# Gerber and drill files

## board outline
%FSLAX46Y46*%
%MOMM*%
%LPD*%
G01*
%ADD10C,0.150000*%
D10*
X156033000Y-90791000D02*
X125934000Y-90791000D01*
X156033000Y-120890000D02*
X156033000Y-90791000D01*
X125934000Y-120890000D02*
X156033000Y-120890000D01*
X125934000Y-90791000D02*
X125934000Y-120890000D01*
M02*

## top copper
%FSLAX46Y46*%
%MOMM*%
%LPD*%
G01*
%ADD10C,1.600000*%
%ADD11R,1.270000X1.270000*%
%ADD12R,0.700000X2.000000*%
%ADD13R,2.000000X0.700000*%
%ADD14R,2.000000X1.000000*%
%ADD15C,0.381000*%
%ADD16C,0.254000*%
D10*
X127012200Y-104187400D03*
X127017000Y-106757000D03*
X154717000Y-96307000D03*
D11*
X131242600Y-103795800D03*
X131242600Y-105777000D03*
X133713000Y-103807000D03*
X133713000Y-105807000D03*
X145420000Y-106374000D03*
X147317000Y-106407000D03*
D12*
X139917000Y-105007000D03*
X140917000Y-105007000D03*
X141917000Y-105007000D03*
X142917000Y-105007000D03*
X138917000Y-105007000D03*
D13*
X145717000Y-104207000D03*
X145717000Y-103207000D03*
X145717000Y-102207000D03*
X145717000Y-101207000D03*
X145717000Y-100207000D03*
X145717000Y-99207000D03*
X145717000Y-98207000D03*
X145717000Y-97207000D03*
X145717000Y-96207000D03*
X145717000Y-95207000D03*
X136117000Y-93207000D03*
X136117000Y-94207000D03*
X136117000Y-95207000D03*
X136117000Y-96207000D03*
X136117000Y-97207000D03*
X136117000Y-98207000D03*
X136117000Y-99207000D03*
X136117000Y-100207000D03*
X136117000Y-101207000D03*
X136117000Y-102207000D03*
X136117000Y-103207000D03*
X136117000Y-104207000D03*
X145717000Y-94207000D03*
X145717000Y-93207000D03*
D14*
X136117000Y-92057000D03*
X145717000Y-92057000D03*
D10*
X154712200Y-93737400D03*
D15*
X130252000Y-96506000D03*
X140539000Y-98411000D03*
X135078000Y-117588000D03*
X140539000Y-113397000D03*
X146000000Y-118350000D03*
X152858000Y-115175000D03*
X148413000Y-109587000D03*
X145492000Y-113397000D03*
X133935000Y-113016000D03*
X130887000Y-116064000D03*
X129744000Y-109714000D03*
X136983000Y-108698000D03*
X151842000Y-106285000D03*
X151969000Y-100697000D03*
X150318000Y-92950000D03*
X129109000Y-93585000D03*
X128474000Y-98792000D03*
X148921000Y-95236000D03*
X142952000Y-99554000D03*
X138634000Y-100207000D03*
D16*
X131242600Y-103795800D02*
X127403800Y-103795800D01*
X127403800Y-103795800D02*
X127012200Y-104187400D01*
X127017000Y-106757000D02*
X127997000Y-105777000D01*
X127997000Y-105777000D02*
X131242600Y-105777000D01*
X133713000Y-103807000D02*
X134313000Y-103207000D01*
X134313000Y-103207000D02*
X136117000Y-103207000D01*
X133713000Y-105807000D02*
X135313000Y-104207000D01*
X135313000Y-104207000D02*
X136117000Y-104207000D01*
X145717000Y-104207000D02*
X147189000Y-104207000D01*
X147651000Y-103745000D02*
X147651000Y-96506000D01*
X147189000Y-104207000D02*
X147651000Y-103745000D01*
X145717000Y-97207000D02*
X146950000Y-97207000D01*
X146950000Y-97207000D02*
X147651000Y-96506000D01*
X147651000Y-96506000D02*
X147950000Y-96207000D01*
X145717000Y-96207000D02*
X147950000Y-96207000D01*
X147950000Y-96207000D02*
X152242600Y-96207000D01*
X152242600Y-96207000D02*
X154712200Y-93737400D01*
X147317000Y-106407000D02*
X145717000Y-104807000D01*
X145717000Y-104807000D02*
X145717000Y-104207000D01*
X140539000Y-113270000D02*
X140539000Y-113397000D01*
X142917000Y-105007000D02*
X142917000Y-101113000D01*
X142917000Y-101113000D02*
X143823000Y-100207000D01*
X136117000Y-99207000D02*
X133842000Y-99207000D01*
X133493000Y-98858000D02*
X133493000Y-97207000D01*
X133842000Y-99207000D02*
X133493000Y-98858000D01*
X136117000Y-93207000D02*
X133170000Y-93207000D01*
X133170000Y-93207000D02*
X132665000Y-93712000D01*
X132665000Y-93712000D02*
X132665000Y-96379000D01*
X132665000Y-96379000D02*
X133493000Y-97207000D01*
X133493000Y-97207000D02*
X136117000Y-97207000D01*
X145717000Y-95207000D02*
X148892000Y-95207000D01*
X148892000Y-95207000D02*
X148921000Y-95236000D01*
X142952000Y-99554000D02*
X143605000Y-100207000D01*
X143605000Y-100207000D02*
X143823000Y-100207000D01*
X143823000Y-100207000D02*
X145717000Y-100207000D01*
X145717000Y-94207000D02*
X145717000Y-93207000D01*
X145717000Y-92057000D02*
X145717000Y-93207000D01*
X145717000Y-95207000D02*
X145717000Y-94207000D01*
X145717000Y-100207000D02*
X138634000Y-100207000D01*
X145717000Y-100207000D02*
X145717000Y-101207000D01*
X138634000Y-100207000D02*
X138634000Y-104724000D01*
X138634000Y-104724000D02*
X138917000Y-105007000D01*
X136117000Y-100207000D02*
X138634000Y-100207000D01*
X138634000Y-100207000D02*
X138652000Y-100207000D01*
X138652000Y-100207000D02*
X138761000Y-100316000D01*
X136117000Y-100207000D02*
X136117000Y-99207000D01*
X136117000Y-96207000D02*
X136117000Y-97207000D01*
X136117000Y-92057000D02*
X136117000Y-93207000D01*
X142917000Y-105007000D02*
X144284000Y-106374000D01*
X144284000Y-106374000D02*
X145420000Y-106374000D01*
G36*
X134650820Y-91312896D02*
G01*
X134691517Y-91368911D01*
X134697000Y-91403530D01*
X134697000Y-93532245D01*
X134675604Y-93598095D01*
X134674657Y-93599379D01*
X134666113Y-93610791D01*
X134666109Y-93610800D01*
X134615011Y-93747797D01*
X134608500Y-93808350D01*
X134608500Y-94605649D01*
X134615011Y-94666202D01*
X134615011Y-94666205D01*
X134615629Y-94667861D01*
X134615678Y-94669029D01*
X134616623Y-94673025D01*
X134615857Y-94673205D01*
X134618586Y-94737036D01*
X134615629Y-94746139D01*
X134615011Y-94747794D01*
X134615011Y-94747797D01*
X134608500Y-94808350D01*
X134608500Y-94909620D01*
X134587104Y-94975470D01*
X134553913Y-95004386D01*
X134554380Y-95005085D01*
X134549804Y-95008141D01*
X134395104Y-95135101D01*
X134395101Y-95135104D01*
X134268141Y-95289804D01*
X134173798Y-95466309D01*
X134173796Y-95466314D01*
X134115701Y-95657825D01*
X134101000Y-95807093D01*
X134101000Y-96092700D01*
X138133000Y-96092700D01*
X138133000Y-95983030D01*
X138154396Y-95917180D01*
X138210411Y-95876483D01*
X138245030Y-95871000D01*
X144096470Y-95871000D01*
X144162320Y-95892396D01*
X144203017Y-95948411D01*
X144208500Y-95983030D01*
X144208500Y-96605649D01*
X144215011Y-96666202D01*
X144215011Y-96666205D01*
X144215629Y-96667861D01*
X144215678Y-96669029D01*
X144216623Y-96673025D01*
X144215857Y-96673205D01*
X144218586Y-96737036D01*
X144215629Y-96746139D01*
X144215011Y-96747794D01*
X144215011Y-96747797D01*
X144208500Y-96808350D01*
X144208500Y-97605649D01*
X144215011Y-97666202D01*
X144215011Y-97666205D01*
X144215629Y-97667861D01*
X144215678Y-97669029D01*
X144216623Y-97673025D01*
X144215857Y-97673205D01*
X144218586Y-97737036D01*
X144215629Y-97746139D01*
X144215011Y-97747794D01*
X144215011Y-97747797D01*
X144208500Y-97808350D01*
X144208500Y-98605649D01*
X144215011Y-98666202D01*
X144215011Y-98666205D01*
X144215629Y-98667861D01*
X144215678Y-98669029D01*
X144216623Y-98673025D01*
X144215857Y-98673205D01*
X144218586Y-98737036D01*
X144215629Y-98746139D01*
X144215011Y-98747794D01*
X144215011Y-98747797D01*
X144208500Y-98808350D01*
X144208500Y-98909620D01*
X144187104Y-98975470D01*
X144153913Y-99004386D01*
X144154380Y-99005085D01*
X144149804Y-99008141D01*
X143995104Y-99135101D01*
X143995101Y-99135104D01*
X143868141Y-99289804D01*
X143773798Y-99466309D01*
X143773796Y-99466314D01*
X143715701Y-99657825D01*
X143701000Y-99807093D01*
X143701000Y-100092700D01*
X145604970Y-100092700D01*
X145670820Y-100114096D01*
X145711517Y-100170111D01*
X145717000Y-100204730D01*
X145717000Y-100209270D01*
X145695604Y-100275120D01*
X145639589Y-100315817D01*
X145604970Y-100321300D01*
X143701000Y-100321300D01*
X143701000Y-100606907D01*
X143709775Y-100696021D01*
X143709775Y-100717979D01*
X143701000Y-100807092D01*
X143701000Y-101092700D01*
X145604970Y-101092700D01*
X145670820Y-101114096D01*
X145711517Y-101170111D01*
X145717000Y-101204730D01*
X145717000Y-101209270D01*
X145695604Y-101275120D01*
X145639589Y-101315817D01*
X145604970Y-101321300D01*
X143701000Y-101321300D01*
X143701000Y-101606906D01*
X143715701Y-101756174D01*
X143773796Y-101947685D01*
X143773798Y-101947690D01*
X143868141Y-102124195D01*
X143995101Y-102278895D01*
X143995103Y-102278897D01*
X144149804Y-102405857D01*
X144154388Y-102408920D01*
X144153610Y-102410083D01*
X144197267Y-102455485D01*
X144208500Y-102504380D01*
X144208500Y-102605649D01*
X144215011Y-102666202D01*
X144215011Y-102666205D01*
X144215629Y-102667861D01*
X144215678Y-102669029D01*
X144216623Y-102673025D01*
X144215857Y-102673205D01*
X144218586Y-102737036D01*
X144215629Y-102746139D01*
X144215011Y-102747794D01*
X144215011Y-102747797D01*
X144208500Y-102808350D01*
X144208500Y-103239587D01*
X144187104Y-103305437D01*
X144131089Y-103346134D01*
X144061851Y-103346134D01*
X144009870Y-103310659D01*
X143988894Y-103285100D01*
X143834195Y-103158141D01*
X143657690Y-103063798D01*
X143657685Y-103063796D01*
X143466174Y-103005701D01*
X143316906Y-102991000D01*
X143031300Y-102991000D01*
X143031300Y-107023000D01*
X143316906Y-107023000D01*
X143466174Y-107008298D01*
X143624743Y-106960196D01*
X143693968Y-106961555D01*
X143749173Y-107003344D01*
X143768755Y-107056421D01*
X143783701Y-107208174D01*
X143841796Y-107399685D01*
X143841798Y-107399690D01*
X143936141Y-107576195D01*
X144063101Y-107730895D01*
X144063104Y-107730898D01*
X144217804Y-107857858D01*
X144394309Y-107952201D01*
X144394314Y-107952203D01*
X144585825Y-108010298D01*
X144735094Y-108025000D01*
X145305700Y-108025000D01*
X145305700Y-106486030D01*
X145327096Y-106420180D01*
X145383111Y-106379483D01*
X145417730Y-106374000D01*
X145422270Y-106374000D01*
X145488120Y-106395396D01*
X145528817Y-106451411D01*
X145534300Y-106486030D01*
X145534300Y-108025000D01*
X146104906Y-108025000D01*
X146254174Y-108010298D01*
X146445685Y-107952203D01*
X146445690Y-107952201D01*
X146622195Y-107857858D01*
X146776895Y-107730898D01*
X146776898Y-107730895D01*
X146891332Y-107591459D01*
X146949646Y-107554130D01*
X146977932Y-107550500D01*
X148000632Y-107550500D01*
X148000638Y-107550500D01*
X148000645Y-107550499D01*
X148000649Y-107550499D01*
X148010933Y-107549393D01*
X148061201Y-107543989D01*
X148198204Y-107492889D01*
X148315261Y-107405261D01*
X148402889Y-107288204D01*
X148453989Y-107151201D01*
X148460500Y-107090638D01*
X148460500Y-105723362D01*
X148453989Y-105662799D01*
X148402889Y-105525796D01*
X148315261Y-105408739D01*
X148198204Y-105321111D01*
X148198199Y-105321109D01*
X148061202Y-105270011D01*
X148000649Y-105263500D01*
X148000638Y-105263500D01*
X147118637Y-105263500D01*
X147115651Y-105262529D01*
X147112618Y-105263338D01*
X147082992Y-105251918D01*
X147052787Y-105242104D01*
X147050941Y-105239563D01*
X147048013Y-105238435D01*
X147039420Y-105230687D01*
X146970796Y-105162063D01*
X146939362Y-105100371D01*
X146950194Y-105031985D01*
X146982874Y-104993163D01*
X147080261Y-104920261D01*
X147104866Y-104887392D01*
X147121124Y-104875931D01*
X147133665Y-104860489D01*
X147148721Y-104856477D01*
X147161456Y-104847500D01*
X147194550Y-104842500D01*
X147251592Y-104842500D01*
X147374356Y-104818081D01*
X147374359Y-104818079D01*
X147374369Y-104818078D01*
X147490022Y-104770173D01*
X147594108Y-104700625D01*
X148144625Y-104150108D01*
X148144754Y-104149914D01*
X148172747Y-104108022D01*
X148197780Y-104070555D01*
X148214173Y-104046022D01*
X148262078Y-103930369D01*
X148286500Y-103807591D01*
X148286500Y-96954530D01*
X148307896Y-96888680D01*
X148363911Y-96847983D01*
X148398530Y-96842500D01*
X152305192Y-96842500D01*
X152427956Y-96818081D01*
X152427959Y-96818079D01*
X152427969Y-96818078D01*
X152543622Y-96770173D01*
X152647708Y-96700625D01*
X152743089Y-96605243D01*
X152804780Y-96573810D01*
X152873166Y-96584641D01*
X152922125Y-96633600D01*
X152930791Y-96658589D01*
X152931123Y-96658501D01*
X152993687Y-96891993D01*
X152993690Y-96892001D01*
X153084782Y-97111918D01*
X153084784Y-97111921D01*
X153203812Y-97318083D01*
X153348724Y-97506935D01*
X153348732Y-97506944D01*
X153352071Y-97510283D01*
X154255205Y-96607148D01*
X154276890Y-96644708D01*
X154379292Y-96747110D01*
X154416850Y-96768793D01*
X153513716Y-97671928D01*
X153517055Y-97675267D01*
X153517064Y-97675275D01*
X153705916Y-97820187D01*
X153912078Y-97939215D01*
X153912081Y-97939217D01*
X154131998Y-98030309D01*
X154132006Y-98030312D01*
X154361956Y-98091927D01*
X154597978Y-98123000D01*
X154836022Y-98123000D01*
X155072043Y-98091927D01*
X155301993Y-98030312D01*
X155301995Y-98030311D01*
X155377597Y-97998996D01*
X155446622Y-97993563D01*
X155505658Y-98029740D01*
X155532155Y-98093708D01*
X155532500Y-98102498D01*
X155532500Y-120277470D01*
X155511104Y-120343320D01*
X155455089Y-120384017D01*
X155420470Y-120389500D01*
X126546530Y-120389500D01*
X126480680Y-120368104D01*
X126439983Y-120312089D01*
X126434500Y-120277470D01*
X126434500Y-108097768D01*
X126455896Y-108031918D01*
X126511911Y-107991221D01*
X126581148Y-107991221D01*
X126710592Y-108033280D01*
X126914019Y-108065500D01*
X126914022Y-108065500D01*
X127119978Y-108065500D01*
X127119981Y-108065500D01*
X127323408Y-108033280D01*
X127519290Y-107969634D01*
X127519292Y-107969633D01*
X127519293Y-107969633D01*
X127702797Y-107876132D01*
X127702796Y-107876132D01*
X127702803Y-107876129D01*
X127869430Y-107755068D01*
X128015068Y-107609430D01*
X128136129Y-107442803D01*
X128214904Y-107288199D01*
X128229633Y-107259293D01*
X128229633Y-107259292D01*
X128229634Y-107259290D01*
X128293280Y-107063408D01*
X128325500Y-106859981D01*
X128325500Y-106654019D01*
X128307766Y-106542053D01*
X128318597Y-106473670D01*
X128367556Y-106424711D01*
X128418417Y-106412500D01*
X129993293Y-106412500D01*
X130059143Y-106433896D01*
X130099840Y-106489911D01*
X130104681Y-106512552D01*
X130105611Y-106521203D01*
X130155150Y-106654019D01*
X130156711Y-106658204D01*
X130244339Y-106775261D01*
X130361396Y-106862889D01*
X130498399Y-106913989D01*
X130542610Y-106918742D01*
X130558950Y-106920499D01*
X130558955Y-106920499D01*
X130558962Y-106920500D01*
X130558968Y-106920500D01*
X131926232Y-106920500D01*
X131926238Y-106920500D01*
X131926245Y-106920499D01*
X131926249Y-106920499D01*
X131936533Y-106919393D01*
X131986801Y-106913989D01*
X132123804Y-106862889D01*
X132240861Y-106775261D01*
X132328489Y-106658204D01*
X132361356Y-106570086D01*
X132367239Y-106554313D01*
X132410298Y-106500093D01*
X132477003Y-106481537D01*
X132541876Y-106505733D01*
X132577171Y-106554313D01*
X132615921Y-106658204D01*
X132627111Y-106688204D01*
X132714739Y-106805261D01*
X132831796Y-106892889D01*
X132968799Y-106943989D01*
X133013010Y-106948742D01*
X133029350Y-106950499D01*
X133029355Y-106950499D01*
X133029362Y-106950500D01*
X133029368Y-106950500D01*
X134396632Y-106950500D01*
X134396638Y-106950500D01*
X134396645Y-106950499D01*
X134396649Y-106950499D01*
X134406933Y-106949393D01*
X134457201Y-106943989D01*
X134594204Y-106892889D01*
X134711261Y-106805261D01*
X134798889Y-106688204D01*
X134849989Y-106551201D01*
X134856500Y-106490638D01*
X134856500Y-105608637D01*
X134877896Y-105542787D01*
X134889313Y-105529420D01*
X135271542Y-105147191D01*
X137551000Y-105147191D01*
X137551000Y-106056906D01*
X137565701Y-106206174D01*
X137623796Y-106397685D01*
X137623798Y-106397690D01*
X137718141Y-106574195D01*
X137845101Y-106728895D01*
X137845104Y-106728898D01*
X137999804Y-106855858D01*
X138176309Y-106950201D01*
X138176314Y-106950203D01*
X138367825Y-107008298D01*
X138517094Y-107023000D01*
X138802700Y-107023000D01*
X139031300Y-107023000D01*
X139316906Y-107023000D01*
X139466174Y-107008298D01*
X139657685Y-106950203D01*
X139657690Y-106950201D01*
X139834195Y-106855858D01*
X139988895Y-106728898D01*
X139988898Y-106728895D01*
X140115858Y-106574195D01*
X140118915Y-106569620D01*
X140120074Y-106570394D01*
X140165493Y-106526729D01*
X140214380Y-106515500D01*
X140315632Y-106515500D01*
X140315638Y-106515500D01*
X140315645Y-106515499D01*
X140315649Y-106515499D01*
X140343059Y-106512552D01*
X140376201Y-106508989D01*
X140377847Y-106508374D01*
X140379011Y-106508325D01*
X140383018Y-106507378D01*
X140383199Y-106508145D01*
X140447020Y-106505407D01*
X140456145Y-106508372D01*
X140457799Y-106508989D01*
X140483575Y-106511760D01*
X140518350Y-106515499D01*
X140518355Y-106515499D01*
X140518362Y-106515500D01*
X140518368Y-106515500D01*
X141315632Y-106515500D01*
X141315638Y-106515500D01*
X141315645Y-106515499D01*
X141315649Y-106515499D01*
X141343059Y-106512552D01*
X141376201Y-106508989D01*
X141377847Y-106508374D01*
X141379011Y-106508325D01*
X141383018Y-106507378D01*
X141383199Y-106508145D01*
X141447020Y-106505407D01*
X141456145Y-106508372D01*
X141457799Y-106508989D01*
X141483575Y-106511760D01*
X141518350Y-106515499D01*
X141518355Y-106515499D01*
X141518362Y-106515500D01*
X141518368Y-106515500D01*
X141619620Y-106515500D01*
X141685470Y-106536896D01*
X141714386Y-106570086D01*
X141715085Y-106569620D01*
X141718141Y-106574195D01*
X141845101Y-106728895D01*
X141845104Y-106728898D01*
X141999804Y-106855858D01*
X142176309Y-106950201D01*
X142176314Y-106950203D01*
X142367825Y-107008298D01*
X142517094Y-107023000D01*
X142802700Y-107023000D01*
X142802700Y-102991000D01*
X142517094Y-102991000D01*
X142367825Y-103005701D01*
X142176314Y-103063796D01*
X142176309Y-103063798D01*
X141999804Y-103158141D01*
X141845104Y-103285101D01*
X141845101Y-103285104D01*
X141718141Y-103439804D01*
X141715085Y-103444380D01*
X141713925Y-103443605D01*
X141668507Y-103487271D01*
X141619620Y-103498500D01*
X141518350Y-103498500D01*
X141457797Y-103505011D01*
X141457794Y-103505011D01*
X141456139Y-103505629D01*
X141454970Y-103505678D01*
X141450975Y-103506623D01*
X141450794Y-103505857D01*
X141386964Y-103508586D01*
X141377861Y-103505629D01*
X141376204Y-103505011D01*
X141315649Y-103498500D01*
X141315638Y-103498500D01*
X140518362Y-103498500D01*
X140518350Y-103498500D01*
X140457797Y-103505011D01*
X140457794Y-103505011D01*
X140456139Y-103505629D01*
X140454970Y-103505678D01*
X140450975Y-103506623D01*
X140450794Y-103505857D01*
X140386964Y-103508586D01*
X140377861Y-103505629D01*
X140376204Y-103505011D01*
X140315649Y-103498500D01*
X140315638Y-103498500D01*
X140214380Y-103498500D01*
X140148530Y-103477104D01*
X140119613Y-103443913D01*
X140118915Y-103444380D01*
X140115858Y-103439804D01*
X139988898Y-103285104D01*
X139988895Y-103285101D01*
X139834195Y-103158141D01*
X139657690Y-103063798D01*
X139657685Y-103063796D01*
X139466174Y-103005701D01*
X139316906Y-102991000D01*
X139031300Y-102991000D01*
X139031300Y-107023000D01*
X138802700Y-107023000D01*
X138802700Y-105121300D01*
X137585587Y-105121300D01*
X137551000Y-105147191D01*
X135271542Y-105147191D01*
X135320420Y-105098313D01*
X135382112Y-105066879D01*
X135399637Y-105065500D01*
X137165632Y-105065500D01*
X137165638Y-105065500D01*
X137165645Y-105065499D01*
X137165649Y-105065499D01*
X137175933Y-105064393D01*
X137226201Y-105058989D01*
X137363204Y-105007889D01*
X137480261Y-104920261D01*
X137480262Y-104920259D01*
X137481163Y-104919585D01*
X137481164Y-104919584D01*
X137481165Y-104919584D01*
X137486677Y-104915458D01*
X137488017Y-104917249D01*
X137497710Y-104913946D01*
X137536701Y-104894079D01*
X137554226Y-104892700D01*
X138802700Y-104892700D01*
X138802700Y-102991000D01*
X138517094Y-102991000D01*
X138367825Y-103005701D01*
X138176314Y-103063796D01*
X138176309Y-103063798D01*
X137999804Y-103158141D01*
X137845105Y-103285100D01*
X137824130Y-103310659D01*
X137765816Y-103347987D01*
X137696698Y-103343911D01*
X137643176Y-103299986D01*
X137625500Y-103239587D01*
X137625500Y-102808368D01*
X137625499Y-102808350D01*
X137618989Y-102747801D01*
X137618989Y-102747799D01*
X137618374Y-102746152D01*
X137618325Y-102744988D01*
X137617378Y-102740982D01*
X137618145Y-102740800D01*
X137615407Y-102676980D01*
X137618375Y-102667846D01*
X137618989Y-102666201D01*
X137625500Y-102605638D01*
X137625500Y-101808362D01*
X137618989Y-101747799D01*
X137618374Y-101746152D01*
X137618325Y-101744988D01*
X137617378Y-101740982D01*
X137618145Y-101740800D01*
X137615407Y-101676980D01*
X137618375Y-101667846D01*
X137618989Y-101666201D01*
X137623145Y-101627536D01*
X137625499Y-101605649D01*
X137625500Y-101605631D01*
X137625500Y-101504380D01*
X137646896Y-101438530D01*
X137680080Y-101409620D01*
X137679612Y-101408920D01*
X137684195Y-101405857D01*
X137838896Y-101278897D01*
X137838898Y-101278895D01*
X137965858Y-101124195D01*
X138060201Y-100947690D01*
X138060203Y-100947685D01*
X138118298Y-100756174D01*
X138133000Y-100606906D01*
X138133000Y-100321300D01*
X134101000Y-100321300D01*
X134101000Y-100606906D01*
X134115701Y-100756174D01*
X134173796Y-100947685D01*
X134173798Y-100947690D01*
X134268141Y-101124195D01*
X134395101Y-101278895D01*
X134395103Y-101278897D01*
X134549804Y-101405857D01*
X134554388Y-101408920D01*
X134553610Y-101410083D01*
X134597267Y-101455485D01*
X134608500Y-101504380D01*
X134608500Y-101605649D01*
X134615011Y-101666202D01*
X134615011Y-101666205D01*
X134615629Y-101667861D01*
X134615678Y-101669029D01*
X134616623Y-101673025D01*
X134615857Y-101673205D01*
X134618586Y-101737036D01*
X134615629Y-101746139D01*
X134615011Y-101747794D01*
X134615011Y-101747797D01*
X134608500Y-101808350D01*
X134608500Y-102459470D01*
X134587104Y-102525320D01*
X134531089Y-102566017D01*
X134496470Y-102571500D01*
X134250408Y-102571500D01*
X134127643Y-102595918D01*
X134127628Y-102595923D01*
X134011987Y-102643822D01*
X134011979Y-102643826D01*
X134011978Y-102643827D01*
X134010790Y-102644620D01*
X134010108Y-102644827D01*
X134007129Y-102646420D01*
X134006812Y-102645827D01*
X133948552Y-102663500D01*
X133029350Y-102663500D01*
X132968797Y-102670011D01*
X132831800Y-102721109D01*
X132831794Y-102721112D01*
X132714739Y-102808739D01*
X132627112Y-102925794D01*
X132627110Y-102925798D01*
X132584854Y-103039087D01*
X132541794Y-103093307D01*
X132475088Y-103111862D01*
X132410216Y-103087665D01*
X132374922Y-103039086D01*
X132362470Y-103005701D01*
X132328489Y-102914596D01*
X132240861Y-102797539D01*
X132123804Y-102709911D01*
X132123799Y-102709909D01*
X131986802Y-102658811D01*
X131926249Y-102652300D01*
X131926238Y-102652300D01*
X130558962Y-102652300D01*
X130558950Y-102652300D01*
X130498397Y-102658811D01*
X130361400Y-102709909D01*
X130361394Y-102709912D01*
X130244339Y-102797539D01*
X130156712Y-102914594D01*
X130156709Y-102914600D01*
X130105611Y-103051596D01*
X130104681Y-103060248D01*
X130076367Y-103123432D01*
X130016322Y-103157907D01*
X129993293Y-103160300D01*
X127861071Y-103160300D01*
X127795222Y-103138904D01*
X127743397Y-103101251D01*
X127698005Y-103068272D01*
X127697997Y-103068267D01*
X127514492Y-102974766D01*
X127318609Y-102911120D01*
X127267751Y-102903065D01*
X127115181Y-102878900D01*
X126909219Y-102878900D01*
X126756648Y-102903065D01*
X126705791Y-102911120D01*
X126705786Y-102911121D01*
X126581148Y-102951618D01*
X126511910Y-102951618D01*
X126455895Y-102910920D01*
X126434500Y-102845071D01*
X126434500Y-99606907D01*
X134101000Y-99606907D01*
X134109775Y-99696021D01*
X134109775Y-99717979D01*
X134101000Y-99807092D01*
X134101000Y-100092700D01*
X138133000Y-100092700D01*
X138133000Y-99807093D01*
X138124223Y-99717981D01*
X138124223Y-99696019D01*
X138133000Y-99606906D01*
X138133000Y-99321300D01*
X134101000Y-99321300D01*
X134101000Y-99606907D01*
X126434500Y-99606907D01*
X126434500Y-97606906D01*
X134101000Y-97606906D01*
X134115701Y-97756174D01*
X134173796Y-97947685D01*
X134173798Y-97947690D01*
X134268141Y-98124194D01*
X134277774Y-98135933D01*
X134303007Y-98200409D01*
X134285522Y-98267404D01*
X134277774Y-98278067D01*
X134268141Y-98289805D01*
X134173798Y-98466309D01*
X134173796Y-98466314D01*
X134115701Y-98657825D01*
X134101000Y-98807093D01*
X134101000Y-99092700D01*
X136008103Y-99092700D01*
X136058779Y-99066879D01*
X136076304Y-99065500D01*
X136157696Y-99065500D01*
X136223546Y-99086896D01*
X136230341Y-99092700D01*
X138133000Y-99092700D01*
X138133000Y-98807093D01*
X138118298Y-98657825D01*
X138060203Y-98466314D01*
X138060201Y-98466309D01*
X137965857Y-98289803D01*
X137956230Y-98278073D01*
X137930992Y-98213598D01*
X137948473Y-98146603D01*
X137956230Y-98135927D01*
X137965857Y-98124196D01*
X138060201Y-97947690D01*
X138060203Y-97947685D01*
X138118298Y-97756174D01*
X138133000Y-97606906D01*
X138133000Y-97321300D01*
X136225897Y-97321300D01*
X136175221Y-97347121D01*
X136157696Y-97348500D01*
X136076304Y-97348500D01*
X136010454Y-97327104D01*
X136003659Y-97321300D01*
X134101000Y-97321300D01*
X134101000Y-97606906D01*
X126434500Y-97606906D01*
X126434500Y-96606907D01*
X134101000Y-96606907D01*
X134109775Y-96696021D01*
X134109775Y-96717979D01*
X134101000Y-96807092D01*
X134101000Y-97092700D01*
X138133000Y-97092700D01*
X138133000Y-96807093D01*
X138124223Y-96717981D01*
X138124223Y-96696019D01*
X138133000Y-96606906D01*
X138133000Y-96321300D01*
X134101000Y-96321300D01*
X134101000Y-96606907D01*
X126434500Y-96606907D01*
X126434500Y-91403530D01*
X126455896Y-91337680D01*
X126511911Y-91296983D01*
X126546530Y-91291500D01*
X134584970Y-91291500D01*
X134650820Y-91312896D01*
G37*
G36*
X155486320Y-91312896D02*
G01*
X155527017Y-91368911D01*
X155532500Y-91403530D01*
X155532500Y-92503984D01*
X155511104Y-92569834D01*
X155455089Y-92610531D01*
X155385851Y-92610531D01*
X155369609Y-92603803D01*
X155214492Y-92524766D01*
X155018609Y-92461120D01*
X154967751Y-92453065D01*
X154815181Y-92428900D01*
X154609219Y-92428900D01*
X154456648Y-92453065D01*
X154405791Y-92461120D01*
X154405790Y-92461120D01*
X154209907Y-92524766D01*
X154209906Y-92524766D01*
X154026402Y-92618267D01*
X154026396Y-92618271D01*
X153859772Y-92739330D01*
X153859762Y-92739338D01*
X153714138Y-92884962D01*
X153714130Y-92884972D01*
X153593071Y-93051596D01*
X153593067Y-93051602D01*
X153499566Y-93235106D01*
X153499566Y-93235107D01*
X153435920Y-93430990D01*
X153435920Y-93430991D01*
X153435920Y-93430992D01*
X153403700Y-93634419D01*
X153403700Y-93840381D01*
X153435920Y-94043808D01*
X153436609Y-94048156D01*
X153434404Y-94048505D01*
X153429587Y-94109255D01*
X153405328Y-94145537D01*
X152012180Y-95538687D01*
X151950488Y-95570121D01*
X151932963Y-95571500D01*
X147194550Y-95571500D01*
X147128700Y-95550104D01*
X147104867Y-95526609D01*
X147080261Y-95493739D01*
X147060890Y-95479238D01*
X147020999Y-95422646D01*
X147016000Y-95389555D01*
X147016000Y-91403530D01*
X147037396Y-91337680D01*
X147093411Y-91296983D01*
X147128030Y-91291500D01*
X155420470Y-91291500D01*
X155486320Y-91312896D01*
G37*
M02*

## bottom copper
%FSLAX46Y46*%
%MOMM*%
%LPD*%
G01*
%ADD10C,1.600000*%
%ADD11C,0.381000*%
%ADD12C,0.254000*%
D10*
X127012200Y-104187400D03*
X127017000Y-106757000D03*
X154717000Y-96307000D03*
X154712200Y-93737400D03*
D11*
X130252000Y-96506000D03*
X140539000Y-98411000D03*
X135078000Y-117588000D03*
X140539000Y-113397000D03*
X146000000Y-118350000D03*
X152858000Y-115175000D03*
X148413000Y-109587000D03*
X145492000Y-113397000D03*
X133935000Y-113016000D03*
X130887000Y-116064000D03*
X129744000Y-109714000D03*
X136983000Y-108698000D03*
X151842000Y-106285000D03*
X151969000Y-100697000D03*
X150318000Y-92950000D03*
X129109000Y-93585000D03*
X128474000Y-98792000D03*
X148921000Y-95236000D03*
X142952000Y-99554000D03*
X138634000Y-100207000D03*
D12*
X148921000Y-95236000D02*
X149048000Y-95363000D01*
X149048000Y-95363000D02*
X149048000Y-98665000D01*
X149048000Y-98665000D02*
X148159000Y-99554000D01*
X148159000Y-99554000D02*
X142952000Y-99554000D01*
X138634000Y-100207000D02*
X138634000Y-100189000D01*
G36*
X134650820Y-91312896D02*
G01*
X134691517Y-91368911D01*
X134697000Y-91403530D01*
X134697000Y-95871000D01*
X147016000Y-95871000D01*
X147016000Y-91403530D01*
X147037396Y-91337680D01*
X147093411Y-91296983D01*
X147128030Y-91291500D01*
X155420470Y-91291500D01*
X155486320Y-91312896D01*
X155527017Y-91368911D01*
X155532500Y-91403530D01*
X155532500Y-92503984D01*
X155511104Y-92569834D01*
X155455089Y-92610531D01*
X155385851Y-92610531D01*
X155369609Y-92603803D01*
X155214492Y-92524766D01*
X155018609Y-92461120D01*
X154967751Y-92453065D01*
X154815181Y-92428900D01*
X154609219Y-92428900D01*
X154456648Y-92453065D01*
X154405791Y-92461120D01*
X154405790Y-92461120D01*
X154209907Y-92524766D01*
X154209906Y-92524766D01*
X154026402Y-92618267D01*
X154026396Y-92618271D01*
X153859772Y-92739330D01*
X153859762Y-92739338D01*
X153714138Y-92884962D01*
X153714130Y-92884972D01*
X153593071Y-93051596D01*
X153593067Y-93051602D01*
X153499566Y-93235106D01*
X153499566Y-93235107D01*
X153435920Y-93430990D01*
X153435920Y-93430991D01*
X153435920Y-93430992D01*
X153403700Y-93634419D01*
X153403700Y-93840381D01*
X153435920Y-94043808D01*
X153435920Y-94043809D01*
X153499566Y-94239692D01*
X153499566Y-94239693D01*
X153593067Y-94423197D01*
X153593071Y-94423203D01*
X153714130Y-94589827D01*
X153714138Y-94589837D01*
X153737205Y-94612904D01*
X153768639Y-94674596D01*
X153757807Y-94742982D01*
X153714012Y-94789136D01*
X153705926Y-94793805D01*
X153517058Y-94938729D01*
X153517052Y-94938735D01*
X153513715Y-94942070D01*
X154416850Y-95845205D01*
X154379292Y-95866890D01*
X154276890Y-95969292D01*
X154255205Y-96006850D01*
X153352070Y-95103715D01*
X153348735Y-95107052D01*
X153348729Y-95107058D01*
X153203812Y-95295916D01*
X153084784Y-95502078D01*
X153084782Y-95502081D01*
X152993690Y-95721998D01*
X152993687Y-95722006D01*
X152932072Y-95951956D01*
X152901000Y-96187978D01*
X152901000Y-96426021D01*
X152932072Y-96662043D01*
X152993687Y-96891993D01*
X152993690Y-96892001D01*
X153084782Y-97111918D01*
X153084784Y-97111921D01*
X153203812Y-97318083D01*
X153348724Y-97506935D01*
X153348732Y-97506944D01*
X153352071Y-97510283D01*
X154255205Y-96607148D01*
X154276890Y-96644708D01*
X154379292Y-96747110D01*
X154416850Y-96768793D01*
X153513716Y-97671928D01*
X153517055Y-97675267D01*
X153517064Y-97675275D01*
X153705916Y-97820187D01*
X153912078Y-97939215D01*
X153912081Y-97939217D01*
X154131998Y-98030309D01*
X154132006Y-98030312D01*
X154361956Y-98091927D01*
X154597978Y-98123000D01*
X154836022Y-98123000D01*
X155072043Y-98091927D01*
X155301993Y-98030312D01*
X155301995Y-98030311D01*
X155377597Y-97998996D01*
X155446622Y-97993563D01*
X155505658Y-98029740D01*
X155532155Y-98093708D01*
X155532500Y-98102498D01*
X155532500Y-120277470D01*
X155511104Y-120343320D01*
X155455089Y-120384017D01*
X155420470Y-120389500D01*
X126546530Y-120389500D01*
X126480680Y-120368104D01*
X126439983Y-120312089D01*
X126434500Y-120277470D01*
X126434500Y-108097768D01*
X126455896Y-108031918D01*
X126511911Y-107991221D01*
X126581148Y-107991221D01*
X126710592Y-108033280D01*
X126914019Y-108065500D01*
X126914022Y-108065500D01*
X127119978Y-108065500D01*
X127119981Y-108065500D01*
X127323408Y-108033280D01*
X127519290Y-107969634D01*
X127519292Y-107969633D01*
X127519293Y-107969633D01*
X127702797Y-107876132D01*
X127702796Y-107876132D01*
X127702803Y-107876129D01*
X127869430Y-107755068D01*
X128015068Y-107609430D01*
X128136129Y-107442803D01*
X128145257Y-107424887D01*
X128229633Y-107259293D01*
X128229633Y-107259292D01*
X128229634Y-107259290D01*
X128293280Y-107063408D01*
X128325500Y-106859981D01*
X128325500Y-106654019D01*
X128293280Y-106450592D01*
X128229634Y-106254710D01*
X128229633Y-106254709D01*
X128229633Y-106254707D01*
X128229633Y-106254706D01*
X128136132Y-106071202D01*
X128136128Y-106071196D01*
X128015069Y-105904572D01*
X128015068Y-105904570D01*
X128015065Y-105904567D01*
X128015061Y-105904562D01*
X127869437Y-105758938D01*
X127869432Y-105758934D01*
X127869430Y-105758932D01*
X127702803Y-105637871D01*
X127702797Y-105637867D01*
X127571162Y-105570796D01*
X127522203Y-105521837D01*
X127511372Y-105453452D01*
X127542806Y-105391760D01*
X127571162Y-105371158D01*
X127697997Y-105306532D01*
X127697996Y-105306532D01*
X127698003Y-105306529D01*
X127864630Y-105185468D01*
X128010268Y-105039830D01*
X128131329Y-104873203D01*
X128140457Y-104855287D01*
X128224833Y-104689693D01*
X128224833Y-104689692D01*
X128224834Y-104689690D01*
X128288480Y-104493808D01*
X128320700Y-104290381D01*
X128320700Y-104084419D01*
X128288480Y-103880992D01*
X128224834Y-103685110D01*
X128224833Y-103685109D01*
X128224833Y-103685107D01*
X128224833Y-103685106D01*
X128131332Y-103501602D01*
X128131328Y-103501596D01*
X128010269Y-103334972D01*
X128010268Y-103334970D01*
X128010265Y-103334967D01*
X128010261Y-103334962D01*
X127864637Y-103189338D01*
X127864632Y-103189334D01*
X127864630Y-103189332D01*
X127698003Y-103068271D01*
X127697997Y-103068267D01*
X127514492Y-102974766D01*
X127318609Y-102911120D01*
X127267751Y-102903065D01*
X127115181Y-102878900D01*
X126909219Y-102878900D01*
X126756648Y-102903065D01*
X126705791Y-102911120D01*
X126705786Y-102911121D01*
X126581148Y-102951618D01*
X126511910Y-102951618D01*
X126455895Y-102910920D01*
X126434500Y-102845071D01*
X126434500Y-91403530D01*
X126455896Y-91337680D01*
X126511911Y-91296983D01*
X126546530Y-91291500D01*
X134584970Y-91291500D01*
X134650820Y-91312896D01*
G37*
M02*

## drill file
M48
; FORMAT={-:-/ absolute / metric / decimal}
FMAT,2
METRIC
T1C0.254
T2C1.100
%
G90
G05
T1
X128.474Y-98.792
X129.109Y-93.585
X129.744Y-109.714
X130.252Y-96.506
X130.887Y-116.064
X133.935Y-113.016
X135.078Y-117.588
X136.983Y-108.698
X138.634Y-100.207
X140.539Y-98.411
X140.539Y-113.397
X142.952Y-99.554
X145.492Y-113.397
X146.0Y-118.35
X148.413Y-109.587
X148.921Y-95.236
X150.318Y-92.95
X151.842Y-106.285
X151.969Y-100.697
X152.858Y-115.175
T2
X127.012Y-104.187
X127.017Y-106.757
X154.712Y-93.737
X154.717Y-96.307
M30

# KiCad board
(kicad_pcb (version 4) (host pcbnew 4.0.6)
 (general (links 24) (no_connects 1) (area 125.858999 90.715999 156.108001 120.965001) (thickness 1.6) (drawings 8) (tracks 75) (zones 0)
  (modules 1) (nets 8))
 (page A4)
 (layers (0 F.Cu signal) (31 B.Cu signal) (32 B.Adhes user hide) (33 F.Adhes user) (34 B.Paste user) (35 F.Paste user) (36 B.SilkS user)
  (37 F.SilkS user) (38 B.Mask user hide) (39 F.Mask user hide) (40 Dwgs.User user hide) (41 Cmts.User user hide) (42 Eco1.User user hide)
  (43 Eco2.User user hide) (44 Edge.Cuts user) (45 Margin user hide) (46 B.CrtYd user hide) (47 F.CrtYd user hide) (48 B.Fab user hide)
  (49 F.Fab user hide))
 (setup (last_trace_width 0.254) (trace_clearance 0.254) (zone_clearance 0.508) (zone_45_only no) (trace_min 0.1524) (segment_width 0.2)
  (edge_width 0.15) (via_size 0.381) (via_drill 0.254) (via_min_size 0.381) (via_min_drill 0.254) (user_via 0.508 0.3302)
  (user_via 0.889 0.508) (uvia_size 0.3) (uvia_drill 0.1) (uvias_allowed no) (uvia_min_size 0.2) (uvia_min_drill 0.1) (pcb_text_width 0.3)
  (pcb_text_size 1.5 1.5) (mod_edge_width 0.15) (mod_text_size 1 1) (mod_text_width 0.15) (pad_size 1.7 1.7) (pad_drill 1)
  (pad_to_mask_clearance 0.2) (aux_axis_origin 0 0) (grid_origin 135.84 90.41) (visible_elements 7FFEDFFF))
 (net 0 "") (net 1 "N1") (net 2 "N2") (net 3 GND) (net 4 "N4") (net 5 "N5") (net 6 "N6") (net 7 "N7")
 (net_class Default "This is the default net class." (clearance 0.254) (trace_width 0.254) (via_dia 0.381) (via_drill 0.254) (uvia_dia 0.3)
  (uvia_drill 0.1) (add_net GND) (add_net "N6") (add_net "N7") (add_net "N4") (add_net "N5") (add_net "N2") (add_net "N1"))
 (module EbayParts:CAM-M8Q (layer F.Cu) (at 135.967 91.807)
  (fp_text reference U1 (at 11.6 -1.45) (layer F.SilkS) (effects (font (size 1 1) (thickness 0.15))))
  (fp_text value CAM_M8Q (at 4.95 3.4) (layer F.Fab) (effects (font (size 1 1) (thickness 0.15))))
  (pad 62 thru_hole circle (at -8.9548 12.3804) (size 1.6 1.6) (drill 1.1) (layers *.Cu *.Mask) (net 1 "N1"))
  (pad 63 thru_hole circle (at -8.95 14.95) (size 1.6 1.6) (drill 1.1) (layers *.Cu *.Mask) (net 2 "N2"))
  (pad 61 thru_hole circle (at 18.75 4.5) (size 1.6 1.6) (drill 1.1) (layers *.Cu *.Mask) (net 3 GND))
  (pad 56 smd rect (at -4.7244 11.9888) (size 1.27 1.27) (layers F.Cu F.Paste F.Mask) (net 1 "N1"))
  (pad 54 smd rect (at -4.7244 13.97) (size 1.27 1.27) (layers F.Cu F.Paste F.Mask) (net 2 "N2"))
  (pad 55 smd rect (at -2.254 12) (size 1.27 1.27) (layers F.Cu F.Paste F.Mask) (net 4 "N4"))
  (pad 53 smd rect (at -2.254 14) (size 1.27 1.27) (layers F.Cu F.Paste F.Mask) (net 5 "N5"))
  (pad 50 smd rect (at 9.453 14.567) (size 1.27 1.27) (layers F.Cu F.Paste F.Mask) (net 3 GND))
  (pad 51 smd rect (at 11.35 14.6) (size 1.27 1.27) (layers F.Cu F.Paste F.Mask) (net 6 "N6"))
  (pad 28 smd rect (at 3.95 13.2) (size 0.7 2) (layers F.Cu F.Paste F.Mask))
  (pad 29 smd rect (at 4.95 13.2) (size 0.7 2) (layers F.Cu F.Paste F.Mask))
  (pad 30 smd rect (at 5.95 13.2) (size 0.7 2) (layers F.Cu F.Paste F.Mask))
  (pad 31 smd rect (at 6.95 13.2) (size 0.7 2) (layers F.Cu F.Paste F.Mask) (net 3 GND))
  (pad 27 smd rect (at 2.95 13.2) (size 0.7 2) (layers F.Cu F.Paste F.Mask) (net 3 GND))
  (pad 1 smd rect (at 9.75 12.4) (size 2 0.7) (layers F.Cu F.Paste F.Mask) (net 6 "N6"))
  (pad 2 smd rect (at 9.75 11.4) (size 2 0.7) (layers F.Cu F.Paste F.Mask))
  (pad 3 smd rect (at 9.75 10.4) (size 2 0.7) (layers F.Cu F.Paste F.Mask))
  (pad 4 smd rect (at 9.75 9.4) (size 2 0.7) (layers F.Cu F.Paste F.Mask) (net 3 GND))
  (pad 5 smd rect (at 9.75 8.4) (size 2 0.7) (layers F.Cu F.Paste F.Mask) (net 3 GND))
  (pad 6 smd rect (at 9.75 7.4) (size 2 0.7) (layers F.Cu F.Paste F.Mask))
  (pad 7 smd rect (at 9.75 6.4) (size 2 0.7) (layers F.Cu F.Paste F.Mask))
  (pad 8 smd rect (at 9.75 5.4) (size 2 0.7) (layers F.Cu F.Paste F.Mask) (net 6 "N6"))
  (pad 9 smd rect (at 9.75 4.4) (size 2 0.7) (layers F.Cu F.Paste F.Mask) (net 6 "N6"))
  (pad 10 smd rect (at 9.75 3.4) (size 2 0.7) (layers F.Cu F.Paste F.Mask) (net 3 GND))
  (pad 15 smd rect (at 0.15 1.4) (size 2 0.7) (layers F.Cu F.Paste F.Mask) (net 3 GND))
  (pad 16 smd rect (at 0.15 2.4) (size 2 0.7) (layers F.Cu F.Paste F.Mask) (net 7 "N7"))
  (pad 17 smd rect (at 0.15 3.4) (size 2 0.7) (layers F.Cu F.Paste F.Mask) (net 7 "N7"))
  (pad 18 smd rect (at 0.15 4.4) (size 2 0.7) (layers F.Cu F.Paste F.Mask) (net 3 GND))
  (pad 19 smd rect (at 0.15 5.4) (size 2 0.7) (layers F.Cu F.Paste F.Mask) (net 3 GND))
  (pad 20 smd rect (at 0.15 6.4) (size 2 0.7) (layers F.Cu F.Paste F.Mask))
  (pad 21 smd rect (at 0.15 7.4) (size 2 0.7) (layers F.Cu F.Paste F.Mask) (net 3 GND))
  (pad 22 smd rect (at 0.15 8.4) (size 2 0.7) (layers F.Cu F.Paste F.Mask) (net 3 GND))
  (pad 23 smd rect (at 0.15 9.4) (size 2 0.7) (layers F.Cu F.Paste F.Mask))
  (pad 24 smd rect (at 0.15 10.4) (size 2 0.7) (layers F.Cu F.Paste F.Mask))
  (pad 25 smd rect (at 0.15 11.4) (size 2 0.7) (layers F.Cu F.Paste F.Mask) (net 4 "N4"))
  (pad 26 smd rect (at 0.15 12.4) (size 2 0.7) (layers F.Cu F.Paste F.Mask) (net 5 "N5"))
  (pad 11 smd rect (at 9.75 2.4) (size 2 0.7) (layers F.Cu F.Paste F.Mask) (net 3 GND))
  (pad 12 smd rect (at 9.75 1.4) (size 2 0.7) (layers F.Cu F.Paste F.Mask) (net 3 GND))
  (pad 14 smd rect (at 0.15 0.25) (size 2 1) (layers F.Cu F.Paste F.Mask) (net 3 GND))
  (pad 13 smd rect (at 9.75 0.25) (size 2 1) (layers F.Cu F.Paste F.Mask) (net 3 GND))
  (pad 60 thru_hole circle (at 18.7452 1.9304) (size 1.6 1.6) (drill 1.1) (layers *.Cu *.Mask) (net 6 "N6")))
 (gr_line (start 156.033 90.791) (end 125.934 90.791) (angle 90) (layer Edge.Cuts) (width 0.15))
 (gr_line (start 156.033 120.89) (end 156.033 90.791) (angle 90) (layer Edge.Cuts) (width 0.15))
 (gr_line (start 125.934 120.89) (end 156.033 120.89) (angle 90) (layer Edge.Cuts) (width 0.15))
 (gr_line (start 125.934 90.791) (end 125.934 120.89) (angle 90) (layer Edge.Cuts) (width 0.15))
 (segment (start 131.2426 103.7958) (end 127.4038 103.7958) (width 0.254) (layer F.Cu) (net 1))
 (segment (start 127.4038 103.7958) (end 127.0122 104.1874) (width 0.254) (layer F.Cu) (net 1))
 (segment (start 127.017 106.757) (end 127.997 105.777) (width 0.254) (layer F.Cu) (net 2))
 (segment (start 127.997 105.777) (end 131.2426 105.777) (width 0.254) (layer F.Cu) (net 2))
 (segment (start 133.713 103.807) (end 134.313 103.207) (width 0.254) (layer F.Cu) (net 4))
 (segment (start 134.313 103.207) (end 136.117 103.207) (width 0.254) (layer F.Cu) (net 4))
 (segment (start 133.713 105.807) (end 135.313 104.207) (width 0.254) (layer F.Cu) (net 5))
 (segment (start 135.313 104.207) (end 136.117 104.207) (width 0.254) (layer F.Cu) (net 5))
 (segment (start 145.717 104.207) (end 147.189 104.207) (width 0.254) (layer F.Cu) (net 6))
 (segment (start 147.651 103.745) (end 147.651 96.506) (width 0.254) (layer F.Cu) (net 6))
 (segment (start 147.189 104.207) (end 147.651 103.745) (width 0.254) (layer F.Cu) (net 6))
 (segment (start 145.717 97.207) (end 146.95 97.207) (width 0.254) (layer F.Cu) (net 6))
 (segment (start 146.95 97.207) (end 147.651 96.506) (width 0.254) (layer F.Cu) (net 6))
 (segment (start 147.651 96.506) (end 147.95 96.207) (width 0.254) (layer F.Cu) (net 6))
 (segment (start 145.717 96.207) (end 147.95 96.207) (width 0.254) (layer F.Cu) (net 6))
 (segment (start 147.95 96.207) (end 152.2426 96.207) (width 0.254) (layer F.Cu) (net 6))
 (segment (start 152.2426 96.207) (end 154.7122 93.7374) (width 0.254) (layer F.Cu) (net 6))
 (segment (start 147.317 106.407) (end 145.717 104.807) (width 0.254) (layer F.Cu) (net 6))
 (segment (start 145.717 104.807) (end 145.717 104.207) (width 0.254) (layer F.Cu) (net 6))
 (via (at 130.252 96.506) (size 0.381) (drill 0.254) (layers F.Cu B.Cu) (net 3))
 (via (at 140.539 98.411) (size 0.381) (drill 0.254) (layers F.Cu B.Cu) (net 3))
 (via (at 135.078 117.588) (size 0.381) (drill 0.254) (layers F.Cu B.Cu) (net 3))
 (segment (start 140.539 113.27) (end 140.539 113.397) (width 0.254) (layer F.Cu) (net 3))
 (via (at 140.539 113.397) (size 0.381) (drill 0.254) (layers F.Cu B.Cu) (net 3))
 (via (at 146 118.35) (size 0.381) (drill 0.254) (layers F.Cu B.Cu) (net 3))
 (via (at 152.858 115.175) (size 0.381) (drill 0.254) (layers F.Cu B.Cu) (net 3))
 (via (at 148.413 109.587) (size 0.381) (drill 0.254) (layers F.Cu B.Cu) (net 3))
 (via (at 145.492 113.397) (size 0.381) (drill 0.254) (layers F.Cu B.Cu) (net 3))
 (via (at 133.935 113.016) (size 0.381) (drill 0.254) (layers F.Cu B.Cu) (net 3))
 (via (at 130.887 116.064) (size 0.381) (drill 0.254) (layers F.Cu B.Cu) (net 3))
 (via (at 129.744 109.714) (size 0.381) (drill 0.254) (layers F.Cu B.Cu) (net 3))
 (via (at 136.983 108.698) (size 0.381) (drill 0.254) (layers F.Cu B.Cu) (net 3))
 (via (at 151.842 106.285) (size 0.381) (drill 0.254) (layers F.Cu B.Cu) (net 3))
 (via (at 151.969 100.697) (size 0.381) (drill 0.254) (layers F.Cu B.Cu) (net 3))
 (via (at 150.318 92.95) (size 0.381) (drill 0.254) (layers F.Cu B.Cu) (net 3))
 (via (at 129.109 93.585) (size 0.381) (drill 0.254) (layers F.Cu B.Cu) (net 3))
 (via (at 128.474 98.792) (size 0.381) (drill 0.254) (layers F.Cu B.Cu) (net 3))
 (segment (start 142.917 105.007) (end 142.917 101.113) (width 0.254) (layer F.Cu) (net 3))
 (segment (start 142.917 101.113) (end 143.823 100.207) (width 0.254) (layer F.Cu) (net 3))
 (segment (start 136.117 99.207) (end 133.842 99.207) (width 0.254) (layer F.Cu) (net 3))
 (segment (start 133.493 98.858) (end 133.493 97.207) (width 0.254) (layer F.Cu) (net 3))
 (segment (start 133.842 99.207) (end 133.493 98.858) (width 0.254) (layer F.Cu) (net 3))
 (segment (start 136.117 93.207) (end 133.17 93.207) (width 0.254) (layer F.Cu) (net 3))
 (segment (start 133.17 93.207) (end 132.665 93.712) (width 0.254) (layer F.Cu) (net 3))
 (segment (start 132.665 93.712) (end 132.665 96.379) (width 0.254) (layer F.Cu) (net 3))
 (segment (start 132.665 96.379) (end 133.493 97.207) (width 0.254) (layer F.Cu) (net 3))
 (segment (start 133.493 97.207) (end 136.117 97.207) (width 0.254) (layer F.Cu) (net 3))
 (segment (start 145.717 95.207) (end 148.892 95.207) (width 0.254) (layer F.Cu) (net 3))
 (segment (start 148.892 95.207) (end 148.921 95.236) (width 0.254) (layer F.Cu) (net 3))
 (via (at 148.921 95.236) (size 0.381) (drill 0.254) (layers F.Cu B.Cu) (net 3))
 (segment (start 148.921 95.236) (end 149.048 95.363) (width 0.254) (layer B.Cu) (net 3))
 (segment (start 149.048 95.363) (end 149.048 98.665) (width 0.254) (layer B.Cu) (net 3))
 (segment (start 149.048 98.665) (end 148.159 99.554) (width 0.254) (layer B.Cu) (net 3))
 (segment (start 148.159 99.554) (end 142.952 99.554) (width 0.254) (layer B.Cu) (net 3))
 (via (at 142.952 99.554) (size 0.381) (drill 0.254) (layers F.Cu B.Cu) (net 3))
 (segment (start 142.952 99.554) (end 143.605 100.207) (width 0.254) (layer F.Cu) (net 3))
 (segment (start 143.605 100.207) (end 143.823 100.207) (width 0.254) (layer F.Cu) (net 3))
 (segment (start 143.823 100.207) (end 145.717 100.207) (width 0.254) (layer F.Cu) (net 3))
 (segment (start 145.717 94.207) (end 145.717 93.207) (width 0.254) (layer F.Cu) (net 3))
 (segment (start 145.717 92.057) (end 145.717 93.207) (width 0.254) (layer F.Cu) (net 3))
 (segment (start 145.717 95.207) (end 145.717 94.207) (width 0.254) (layer F.Cu) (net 3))
 (segment (start 145.717 100.207) (end 138.634 100.207) (width 0.254) (layer F.Cu) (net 3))
 (segment (start 145.717 100.207) (end 145.717 101.207) (width 0.254) (layer F.Cu) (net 3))
 (segment (start 138.634 100.207) (end 138.634 104.724) (width 0.254) (layer F.Cu) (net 3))
 (segment (start 138.634 104.724) (end 138.917 105.007) (width 0.254) (layer F.Cu) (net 3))
 (via (at 138.634 100.207) (size 0.381) (drill 0.254) (layers F.Cu B.Cu) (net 3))
 (segment (start 138.634 100.207) (end 138.634 100.189) (width 0.254) (layer B.Cu) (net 3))
 (segment (start 136.117 100.207) (end 138.634 100.207) (width 0.254) (layer F.Cu) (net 3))
 (segment (start 138.634 100.207) (end 138.652 100.207) (width 0.254) (layer F.Cu) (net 3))
 (segment (start 138.652 100.207) (end 138.761 100.316) (width 0.254) (layer F.Cu) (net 3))
 (segment (start 136.117 100.207) (end 136.117 99.207) (width 0.254) (layer F.Cu) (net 3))
 (segment (start 136.117 96.207) (end 136.117 97.207) (width 0.254) (layer F.Cu) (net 3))
 (segment (start 136.117 92.057) (end 136.117 93.207) (width 0.254) (layer F.Cu) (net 3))
 (segment (start 142.917 105.007) (end 144.284 106.374) (width 0.254) (layer F.Cu) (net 3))
 (segment (start 144.284 106.374) (end 145.42 106.374) (width 0.254) (layer F.Cu) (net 3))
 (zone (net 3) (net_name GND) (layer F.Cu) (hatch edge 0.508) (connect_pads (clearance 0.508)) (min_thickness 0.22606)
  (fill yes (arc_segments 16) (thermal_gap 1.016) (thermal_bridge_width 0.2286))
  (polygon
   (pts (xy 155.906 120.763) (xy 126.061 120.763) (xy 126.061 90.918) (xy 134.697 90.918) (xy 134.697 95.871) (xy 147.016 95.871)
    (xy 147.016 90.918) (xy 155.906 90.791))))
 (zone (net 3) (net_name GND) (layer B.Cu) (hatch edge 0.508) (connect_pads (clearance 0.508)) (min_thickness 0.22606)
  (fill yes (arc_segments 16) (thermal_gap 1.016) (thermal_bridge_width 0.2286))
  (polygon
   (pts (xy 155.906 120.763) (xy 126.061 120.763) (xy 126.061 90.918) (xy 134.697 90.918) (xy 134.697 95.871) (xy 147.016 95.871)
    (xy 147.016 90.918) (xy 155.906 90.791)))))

